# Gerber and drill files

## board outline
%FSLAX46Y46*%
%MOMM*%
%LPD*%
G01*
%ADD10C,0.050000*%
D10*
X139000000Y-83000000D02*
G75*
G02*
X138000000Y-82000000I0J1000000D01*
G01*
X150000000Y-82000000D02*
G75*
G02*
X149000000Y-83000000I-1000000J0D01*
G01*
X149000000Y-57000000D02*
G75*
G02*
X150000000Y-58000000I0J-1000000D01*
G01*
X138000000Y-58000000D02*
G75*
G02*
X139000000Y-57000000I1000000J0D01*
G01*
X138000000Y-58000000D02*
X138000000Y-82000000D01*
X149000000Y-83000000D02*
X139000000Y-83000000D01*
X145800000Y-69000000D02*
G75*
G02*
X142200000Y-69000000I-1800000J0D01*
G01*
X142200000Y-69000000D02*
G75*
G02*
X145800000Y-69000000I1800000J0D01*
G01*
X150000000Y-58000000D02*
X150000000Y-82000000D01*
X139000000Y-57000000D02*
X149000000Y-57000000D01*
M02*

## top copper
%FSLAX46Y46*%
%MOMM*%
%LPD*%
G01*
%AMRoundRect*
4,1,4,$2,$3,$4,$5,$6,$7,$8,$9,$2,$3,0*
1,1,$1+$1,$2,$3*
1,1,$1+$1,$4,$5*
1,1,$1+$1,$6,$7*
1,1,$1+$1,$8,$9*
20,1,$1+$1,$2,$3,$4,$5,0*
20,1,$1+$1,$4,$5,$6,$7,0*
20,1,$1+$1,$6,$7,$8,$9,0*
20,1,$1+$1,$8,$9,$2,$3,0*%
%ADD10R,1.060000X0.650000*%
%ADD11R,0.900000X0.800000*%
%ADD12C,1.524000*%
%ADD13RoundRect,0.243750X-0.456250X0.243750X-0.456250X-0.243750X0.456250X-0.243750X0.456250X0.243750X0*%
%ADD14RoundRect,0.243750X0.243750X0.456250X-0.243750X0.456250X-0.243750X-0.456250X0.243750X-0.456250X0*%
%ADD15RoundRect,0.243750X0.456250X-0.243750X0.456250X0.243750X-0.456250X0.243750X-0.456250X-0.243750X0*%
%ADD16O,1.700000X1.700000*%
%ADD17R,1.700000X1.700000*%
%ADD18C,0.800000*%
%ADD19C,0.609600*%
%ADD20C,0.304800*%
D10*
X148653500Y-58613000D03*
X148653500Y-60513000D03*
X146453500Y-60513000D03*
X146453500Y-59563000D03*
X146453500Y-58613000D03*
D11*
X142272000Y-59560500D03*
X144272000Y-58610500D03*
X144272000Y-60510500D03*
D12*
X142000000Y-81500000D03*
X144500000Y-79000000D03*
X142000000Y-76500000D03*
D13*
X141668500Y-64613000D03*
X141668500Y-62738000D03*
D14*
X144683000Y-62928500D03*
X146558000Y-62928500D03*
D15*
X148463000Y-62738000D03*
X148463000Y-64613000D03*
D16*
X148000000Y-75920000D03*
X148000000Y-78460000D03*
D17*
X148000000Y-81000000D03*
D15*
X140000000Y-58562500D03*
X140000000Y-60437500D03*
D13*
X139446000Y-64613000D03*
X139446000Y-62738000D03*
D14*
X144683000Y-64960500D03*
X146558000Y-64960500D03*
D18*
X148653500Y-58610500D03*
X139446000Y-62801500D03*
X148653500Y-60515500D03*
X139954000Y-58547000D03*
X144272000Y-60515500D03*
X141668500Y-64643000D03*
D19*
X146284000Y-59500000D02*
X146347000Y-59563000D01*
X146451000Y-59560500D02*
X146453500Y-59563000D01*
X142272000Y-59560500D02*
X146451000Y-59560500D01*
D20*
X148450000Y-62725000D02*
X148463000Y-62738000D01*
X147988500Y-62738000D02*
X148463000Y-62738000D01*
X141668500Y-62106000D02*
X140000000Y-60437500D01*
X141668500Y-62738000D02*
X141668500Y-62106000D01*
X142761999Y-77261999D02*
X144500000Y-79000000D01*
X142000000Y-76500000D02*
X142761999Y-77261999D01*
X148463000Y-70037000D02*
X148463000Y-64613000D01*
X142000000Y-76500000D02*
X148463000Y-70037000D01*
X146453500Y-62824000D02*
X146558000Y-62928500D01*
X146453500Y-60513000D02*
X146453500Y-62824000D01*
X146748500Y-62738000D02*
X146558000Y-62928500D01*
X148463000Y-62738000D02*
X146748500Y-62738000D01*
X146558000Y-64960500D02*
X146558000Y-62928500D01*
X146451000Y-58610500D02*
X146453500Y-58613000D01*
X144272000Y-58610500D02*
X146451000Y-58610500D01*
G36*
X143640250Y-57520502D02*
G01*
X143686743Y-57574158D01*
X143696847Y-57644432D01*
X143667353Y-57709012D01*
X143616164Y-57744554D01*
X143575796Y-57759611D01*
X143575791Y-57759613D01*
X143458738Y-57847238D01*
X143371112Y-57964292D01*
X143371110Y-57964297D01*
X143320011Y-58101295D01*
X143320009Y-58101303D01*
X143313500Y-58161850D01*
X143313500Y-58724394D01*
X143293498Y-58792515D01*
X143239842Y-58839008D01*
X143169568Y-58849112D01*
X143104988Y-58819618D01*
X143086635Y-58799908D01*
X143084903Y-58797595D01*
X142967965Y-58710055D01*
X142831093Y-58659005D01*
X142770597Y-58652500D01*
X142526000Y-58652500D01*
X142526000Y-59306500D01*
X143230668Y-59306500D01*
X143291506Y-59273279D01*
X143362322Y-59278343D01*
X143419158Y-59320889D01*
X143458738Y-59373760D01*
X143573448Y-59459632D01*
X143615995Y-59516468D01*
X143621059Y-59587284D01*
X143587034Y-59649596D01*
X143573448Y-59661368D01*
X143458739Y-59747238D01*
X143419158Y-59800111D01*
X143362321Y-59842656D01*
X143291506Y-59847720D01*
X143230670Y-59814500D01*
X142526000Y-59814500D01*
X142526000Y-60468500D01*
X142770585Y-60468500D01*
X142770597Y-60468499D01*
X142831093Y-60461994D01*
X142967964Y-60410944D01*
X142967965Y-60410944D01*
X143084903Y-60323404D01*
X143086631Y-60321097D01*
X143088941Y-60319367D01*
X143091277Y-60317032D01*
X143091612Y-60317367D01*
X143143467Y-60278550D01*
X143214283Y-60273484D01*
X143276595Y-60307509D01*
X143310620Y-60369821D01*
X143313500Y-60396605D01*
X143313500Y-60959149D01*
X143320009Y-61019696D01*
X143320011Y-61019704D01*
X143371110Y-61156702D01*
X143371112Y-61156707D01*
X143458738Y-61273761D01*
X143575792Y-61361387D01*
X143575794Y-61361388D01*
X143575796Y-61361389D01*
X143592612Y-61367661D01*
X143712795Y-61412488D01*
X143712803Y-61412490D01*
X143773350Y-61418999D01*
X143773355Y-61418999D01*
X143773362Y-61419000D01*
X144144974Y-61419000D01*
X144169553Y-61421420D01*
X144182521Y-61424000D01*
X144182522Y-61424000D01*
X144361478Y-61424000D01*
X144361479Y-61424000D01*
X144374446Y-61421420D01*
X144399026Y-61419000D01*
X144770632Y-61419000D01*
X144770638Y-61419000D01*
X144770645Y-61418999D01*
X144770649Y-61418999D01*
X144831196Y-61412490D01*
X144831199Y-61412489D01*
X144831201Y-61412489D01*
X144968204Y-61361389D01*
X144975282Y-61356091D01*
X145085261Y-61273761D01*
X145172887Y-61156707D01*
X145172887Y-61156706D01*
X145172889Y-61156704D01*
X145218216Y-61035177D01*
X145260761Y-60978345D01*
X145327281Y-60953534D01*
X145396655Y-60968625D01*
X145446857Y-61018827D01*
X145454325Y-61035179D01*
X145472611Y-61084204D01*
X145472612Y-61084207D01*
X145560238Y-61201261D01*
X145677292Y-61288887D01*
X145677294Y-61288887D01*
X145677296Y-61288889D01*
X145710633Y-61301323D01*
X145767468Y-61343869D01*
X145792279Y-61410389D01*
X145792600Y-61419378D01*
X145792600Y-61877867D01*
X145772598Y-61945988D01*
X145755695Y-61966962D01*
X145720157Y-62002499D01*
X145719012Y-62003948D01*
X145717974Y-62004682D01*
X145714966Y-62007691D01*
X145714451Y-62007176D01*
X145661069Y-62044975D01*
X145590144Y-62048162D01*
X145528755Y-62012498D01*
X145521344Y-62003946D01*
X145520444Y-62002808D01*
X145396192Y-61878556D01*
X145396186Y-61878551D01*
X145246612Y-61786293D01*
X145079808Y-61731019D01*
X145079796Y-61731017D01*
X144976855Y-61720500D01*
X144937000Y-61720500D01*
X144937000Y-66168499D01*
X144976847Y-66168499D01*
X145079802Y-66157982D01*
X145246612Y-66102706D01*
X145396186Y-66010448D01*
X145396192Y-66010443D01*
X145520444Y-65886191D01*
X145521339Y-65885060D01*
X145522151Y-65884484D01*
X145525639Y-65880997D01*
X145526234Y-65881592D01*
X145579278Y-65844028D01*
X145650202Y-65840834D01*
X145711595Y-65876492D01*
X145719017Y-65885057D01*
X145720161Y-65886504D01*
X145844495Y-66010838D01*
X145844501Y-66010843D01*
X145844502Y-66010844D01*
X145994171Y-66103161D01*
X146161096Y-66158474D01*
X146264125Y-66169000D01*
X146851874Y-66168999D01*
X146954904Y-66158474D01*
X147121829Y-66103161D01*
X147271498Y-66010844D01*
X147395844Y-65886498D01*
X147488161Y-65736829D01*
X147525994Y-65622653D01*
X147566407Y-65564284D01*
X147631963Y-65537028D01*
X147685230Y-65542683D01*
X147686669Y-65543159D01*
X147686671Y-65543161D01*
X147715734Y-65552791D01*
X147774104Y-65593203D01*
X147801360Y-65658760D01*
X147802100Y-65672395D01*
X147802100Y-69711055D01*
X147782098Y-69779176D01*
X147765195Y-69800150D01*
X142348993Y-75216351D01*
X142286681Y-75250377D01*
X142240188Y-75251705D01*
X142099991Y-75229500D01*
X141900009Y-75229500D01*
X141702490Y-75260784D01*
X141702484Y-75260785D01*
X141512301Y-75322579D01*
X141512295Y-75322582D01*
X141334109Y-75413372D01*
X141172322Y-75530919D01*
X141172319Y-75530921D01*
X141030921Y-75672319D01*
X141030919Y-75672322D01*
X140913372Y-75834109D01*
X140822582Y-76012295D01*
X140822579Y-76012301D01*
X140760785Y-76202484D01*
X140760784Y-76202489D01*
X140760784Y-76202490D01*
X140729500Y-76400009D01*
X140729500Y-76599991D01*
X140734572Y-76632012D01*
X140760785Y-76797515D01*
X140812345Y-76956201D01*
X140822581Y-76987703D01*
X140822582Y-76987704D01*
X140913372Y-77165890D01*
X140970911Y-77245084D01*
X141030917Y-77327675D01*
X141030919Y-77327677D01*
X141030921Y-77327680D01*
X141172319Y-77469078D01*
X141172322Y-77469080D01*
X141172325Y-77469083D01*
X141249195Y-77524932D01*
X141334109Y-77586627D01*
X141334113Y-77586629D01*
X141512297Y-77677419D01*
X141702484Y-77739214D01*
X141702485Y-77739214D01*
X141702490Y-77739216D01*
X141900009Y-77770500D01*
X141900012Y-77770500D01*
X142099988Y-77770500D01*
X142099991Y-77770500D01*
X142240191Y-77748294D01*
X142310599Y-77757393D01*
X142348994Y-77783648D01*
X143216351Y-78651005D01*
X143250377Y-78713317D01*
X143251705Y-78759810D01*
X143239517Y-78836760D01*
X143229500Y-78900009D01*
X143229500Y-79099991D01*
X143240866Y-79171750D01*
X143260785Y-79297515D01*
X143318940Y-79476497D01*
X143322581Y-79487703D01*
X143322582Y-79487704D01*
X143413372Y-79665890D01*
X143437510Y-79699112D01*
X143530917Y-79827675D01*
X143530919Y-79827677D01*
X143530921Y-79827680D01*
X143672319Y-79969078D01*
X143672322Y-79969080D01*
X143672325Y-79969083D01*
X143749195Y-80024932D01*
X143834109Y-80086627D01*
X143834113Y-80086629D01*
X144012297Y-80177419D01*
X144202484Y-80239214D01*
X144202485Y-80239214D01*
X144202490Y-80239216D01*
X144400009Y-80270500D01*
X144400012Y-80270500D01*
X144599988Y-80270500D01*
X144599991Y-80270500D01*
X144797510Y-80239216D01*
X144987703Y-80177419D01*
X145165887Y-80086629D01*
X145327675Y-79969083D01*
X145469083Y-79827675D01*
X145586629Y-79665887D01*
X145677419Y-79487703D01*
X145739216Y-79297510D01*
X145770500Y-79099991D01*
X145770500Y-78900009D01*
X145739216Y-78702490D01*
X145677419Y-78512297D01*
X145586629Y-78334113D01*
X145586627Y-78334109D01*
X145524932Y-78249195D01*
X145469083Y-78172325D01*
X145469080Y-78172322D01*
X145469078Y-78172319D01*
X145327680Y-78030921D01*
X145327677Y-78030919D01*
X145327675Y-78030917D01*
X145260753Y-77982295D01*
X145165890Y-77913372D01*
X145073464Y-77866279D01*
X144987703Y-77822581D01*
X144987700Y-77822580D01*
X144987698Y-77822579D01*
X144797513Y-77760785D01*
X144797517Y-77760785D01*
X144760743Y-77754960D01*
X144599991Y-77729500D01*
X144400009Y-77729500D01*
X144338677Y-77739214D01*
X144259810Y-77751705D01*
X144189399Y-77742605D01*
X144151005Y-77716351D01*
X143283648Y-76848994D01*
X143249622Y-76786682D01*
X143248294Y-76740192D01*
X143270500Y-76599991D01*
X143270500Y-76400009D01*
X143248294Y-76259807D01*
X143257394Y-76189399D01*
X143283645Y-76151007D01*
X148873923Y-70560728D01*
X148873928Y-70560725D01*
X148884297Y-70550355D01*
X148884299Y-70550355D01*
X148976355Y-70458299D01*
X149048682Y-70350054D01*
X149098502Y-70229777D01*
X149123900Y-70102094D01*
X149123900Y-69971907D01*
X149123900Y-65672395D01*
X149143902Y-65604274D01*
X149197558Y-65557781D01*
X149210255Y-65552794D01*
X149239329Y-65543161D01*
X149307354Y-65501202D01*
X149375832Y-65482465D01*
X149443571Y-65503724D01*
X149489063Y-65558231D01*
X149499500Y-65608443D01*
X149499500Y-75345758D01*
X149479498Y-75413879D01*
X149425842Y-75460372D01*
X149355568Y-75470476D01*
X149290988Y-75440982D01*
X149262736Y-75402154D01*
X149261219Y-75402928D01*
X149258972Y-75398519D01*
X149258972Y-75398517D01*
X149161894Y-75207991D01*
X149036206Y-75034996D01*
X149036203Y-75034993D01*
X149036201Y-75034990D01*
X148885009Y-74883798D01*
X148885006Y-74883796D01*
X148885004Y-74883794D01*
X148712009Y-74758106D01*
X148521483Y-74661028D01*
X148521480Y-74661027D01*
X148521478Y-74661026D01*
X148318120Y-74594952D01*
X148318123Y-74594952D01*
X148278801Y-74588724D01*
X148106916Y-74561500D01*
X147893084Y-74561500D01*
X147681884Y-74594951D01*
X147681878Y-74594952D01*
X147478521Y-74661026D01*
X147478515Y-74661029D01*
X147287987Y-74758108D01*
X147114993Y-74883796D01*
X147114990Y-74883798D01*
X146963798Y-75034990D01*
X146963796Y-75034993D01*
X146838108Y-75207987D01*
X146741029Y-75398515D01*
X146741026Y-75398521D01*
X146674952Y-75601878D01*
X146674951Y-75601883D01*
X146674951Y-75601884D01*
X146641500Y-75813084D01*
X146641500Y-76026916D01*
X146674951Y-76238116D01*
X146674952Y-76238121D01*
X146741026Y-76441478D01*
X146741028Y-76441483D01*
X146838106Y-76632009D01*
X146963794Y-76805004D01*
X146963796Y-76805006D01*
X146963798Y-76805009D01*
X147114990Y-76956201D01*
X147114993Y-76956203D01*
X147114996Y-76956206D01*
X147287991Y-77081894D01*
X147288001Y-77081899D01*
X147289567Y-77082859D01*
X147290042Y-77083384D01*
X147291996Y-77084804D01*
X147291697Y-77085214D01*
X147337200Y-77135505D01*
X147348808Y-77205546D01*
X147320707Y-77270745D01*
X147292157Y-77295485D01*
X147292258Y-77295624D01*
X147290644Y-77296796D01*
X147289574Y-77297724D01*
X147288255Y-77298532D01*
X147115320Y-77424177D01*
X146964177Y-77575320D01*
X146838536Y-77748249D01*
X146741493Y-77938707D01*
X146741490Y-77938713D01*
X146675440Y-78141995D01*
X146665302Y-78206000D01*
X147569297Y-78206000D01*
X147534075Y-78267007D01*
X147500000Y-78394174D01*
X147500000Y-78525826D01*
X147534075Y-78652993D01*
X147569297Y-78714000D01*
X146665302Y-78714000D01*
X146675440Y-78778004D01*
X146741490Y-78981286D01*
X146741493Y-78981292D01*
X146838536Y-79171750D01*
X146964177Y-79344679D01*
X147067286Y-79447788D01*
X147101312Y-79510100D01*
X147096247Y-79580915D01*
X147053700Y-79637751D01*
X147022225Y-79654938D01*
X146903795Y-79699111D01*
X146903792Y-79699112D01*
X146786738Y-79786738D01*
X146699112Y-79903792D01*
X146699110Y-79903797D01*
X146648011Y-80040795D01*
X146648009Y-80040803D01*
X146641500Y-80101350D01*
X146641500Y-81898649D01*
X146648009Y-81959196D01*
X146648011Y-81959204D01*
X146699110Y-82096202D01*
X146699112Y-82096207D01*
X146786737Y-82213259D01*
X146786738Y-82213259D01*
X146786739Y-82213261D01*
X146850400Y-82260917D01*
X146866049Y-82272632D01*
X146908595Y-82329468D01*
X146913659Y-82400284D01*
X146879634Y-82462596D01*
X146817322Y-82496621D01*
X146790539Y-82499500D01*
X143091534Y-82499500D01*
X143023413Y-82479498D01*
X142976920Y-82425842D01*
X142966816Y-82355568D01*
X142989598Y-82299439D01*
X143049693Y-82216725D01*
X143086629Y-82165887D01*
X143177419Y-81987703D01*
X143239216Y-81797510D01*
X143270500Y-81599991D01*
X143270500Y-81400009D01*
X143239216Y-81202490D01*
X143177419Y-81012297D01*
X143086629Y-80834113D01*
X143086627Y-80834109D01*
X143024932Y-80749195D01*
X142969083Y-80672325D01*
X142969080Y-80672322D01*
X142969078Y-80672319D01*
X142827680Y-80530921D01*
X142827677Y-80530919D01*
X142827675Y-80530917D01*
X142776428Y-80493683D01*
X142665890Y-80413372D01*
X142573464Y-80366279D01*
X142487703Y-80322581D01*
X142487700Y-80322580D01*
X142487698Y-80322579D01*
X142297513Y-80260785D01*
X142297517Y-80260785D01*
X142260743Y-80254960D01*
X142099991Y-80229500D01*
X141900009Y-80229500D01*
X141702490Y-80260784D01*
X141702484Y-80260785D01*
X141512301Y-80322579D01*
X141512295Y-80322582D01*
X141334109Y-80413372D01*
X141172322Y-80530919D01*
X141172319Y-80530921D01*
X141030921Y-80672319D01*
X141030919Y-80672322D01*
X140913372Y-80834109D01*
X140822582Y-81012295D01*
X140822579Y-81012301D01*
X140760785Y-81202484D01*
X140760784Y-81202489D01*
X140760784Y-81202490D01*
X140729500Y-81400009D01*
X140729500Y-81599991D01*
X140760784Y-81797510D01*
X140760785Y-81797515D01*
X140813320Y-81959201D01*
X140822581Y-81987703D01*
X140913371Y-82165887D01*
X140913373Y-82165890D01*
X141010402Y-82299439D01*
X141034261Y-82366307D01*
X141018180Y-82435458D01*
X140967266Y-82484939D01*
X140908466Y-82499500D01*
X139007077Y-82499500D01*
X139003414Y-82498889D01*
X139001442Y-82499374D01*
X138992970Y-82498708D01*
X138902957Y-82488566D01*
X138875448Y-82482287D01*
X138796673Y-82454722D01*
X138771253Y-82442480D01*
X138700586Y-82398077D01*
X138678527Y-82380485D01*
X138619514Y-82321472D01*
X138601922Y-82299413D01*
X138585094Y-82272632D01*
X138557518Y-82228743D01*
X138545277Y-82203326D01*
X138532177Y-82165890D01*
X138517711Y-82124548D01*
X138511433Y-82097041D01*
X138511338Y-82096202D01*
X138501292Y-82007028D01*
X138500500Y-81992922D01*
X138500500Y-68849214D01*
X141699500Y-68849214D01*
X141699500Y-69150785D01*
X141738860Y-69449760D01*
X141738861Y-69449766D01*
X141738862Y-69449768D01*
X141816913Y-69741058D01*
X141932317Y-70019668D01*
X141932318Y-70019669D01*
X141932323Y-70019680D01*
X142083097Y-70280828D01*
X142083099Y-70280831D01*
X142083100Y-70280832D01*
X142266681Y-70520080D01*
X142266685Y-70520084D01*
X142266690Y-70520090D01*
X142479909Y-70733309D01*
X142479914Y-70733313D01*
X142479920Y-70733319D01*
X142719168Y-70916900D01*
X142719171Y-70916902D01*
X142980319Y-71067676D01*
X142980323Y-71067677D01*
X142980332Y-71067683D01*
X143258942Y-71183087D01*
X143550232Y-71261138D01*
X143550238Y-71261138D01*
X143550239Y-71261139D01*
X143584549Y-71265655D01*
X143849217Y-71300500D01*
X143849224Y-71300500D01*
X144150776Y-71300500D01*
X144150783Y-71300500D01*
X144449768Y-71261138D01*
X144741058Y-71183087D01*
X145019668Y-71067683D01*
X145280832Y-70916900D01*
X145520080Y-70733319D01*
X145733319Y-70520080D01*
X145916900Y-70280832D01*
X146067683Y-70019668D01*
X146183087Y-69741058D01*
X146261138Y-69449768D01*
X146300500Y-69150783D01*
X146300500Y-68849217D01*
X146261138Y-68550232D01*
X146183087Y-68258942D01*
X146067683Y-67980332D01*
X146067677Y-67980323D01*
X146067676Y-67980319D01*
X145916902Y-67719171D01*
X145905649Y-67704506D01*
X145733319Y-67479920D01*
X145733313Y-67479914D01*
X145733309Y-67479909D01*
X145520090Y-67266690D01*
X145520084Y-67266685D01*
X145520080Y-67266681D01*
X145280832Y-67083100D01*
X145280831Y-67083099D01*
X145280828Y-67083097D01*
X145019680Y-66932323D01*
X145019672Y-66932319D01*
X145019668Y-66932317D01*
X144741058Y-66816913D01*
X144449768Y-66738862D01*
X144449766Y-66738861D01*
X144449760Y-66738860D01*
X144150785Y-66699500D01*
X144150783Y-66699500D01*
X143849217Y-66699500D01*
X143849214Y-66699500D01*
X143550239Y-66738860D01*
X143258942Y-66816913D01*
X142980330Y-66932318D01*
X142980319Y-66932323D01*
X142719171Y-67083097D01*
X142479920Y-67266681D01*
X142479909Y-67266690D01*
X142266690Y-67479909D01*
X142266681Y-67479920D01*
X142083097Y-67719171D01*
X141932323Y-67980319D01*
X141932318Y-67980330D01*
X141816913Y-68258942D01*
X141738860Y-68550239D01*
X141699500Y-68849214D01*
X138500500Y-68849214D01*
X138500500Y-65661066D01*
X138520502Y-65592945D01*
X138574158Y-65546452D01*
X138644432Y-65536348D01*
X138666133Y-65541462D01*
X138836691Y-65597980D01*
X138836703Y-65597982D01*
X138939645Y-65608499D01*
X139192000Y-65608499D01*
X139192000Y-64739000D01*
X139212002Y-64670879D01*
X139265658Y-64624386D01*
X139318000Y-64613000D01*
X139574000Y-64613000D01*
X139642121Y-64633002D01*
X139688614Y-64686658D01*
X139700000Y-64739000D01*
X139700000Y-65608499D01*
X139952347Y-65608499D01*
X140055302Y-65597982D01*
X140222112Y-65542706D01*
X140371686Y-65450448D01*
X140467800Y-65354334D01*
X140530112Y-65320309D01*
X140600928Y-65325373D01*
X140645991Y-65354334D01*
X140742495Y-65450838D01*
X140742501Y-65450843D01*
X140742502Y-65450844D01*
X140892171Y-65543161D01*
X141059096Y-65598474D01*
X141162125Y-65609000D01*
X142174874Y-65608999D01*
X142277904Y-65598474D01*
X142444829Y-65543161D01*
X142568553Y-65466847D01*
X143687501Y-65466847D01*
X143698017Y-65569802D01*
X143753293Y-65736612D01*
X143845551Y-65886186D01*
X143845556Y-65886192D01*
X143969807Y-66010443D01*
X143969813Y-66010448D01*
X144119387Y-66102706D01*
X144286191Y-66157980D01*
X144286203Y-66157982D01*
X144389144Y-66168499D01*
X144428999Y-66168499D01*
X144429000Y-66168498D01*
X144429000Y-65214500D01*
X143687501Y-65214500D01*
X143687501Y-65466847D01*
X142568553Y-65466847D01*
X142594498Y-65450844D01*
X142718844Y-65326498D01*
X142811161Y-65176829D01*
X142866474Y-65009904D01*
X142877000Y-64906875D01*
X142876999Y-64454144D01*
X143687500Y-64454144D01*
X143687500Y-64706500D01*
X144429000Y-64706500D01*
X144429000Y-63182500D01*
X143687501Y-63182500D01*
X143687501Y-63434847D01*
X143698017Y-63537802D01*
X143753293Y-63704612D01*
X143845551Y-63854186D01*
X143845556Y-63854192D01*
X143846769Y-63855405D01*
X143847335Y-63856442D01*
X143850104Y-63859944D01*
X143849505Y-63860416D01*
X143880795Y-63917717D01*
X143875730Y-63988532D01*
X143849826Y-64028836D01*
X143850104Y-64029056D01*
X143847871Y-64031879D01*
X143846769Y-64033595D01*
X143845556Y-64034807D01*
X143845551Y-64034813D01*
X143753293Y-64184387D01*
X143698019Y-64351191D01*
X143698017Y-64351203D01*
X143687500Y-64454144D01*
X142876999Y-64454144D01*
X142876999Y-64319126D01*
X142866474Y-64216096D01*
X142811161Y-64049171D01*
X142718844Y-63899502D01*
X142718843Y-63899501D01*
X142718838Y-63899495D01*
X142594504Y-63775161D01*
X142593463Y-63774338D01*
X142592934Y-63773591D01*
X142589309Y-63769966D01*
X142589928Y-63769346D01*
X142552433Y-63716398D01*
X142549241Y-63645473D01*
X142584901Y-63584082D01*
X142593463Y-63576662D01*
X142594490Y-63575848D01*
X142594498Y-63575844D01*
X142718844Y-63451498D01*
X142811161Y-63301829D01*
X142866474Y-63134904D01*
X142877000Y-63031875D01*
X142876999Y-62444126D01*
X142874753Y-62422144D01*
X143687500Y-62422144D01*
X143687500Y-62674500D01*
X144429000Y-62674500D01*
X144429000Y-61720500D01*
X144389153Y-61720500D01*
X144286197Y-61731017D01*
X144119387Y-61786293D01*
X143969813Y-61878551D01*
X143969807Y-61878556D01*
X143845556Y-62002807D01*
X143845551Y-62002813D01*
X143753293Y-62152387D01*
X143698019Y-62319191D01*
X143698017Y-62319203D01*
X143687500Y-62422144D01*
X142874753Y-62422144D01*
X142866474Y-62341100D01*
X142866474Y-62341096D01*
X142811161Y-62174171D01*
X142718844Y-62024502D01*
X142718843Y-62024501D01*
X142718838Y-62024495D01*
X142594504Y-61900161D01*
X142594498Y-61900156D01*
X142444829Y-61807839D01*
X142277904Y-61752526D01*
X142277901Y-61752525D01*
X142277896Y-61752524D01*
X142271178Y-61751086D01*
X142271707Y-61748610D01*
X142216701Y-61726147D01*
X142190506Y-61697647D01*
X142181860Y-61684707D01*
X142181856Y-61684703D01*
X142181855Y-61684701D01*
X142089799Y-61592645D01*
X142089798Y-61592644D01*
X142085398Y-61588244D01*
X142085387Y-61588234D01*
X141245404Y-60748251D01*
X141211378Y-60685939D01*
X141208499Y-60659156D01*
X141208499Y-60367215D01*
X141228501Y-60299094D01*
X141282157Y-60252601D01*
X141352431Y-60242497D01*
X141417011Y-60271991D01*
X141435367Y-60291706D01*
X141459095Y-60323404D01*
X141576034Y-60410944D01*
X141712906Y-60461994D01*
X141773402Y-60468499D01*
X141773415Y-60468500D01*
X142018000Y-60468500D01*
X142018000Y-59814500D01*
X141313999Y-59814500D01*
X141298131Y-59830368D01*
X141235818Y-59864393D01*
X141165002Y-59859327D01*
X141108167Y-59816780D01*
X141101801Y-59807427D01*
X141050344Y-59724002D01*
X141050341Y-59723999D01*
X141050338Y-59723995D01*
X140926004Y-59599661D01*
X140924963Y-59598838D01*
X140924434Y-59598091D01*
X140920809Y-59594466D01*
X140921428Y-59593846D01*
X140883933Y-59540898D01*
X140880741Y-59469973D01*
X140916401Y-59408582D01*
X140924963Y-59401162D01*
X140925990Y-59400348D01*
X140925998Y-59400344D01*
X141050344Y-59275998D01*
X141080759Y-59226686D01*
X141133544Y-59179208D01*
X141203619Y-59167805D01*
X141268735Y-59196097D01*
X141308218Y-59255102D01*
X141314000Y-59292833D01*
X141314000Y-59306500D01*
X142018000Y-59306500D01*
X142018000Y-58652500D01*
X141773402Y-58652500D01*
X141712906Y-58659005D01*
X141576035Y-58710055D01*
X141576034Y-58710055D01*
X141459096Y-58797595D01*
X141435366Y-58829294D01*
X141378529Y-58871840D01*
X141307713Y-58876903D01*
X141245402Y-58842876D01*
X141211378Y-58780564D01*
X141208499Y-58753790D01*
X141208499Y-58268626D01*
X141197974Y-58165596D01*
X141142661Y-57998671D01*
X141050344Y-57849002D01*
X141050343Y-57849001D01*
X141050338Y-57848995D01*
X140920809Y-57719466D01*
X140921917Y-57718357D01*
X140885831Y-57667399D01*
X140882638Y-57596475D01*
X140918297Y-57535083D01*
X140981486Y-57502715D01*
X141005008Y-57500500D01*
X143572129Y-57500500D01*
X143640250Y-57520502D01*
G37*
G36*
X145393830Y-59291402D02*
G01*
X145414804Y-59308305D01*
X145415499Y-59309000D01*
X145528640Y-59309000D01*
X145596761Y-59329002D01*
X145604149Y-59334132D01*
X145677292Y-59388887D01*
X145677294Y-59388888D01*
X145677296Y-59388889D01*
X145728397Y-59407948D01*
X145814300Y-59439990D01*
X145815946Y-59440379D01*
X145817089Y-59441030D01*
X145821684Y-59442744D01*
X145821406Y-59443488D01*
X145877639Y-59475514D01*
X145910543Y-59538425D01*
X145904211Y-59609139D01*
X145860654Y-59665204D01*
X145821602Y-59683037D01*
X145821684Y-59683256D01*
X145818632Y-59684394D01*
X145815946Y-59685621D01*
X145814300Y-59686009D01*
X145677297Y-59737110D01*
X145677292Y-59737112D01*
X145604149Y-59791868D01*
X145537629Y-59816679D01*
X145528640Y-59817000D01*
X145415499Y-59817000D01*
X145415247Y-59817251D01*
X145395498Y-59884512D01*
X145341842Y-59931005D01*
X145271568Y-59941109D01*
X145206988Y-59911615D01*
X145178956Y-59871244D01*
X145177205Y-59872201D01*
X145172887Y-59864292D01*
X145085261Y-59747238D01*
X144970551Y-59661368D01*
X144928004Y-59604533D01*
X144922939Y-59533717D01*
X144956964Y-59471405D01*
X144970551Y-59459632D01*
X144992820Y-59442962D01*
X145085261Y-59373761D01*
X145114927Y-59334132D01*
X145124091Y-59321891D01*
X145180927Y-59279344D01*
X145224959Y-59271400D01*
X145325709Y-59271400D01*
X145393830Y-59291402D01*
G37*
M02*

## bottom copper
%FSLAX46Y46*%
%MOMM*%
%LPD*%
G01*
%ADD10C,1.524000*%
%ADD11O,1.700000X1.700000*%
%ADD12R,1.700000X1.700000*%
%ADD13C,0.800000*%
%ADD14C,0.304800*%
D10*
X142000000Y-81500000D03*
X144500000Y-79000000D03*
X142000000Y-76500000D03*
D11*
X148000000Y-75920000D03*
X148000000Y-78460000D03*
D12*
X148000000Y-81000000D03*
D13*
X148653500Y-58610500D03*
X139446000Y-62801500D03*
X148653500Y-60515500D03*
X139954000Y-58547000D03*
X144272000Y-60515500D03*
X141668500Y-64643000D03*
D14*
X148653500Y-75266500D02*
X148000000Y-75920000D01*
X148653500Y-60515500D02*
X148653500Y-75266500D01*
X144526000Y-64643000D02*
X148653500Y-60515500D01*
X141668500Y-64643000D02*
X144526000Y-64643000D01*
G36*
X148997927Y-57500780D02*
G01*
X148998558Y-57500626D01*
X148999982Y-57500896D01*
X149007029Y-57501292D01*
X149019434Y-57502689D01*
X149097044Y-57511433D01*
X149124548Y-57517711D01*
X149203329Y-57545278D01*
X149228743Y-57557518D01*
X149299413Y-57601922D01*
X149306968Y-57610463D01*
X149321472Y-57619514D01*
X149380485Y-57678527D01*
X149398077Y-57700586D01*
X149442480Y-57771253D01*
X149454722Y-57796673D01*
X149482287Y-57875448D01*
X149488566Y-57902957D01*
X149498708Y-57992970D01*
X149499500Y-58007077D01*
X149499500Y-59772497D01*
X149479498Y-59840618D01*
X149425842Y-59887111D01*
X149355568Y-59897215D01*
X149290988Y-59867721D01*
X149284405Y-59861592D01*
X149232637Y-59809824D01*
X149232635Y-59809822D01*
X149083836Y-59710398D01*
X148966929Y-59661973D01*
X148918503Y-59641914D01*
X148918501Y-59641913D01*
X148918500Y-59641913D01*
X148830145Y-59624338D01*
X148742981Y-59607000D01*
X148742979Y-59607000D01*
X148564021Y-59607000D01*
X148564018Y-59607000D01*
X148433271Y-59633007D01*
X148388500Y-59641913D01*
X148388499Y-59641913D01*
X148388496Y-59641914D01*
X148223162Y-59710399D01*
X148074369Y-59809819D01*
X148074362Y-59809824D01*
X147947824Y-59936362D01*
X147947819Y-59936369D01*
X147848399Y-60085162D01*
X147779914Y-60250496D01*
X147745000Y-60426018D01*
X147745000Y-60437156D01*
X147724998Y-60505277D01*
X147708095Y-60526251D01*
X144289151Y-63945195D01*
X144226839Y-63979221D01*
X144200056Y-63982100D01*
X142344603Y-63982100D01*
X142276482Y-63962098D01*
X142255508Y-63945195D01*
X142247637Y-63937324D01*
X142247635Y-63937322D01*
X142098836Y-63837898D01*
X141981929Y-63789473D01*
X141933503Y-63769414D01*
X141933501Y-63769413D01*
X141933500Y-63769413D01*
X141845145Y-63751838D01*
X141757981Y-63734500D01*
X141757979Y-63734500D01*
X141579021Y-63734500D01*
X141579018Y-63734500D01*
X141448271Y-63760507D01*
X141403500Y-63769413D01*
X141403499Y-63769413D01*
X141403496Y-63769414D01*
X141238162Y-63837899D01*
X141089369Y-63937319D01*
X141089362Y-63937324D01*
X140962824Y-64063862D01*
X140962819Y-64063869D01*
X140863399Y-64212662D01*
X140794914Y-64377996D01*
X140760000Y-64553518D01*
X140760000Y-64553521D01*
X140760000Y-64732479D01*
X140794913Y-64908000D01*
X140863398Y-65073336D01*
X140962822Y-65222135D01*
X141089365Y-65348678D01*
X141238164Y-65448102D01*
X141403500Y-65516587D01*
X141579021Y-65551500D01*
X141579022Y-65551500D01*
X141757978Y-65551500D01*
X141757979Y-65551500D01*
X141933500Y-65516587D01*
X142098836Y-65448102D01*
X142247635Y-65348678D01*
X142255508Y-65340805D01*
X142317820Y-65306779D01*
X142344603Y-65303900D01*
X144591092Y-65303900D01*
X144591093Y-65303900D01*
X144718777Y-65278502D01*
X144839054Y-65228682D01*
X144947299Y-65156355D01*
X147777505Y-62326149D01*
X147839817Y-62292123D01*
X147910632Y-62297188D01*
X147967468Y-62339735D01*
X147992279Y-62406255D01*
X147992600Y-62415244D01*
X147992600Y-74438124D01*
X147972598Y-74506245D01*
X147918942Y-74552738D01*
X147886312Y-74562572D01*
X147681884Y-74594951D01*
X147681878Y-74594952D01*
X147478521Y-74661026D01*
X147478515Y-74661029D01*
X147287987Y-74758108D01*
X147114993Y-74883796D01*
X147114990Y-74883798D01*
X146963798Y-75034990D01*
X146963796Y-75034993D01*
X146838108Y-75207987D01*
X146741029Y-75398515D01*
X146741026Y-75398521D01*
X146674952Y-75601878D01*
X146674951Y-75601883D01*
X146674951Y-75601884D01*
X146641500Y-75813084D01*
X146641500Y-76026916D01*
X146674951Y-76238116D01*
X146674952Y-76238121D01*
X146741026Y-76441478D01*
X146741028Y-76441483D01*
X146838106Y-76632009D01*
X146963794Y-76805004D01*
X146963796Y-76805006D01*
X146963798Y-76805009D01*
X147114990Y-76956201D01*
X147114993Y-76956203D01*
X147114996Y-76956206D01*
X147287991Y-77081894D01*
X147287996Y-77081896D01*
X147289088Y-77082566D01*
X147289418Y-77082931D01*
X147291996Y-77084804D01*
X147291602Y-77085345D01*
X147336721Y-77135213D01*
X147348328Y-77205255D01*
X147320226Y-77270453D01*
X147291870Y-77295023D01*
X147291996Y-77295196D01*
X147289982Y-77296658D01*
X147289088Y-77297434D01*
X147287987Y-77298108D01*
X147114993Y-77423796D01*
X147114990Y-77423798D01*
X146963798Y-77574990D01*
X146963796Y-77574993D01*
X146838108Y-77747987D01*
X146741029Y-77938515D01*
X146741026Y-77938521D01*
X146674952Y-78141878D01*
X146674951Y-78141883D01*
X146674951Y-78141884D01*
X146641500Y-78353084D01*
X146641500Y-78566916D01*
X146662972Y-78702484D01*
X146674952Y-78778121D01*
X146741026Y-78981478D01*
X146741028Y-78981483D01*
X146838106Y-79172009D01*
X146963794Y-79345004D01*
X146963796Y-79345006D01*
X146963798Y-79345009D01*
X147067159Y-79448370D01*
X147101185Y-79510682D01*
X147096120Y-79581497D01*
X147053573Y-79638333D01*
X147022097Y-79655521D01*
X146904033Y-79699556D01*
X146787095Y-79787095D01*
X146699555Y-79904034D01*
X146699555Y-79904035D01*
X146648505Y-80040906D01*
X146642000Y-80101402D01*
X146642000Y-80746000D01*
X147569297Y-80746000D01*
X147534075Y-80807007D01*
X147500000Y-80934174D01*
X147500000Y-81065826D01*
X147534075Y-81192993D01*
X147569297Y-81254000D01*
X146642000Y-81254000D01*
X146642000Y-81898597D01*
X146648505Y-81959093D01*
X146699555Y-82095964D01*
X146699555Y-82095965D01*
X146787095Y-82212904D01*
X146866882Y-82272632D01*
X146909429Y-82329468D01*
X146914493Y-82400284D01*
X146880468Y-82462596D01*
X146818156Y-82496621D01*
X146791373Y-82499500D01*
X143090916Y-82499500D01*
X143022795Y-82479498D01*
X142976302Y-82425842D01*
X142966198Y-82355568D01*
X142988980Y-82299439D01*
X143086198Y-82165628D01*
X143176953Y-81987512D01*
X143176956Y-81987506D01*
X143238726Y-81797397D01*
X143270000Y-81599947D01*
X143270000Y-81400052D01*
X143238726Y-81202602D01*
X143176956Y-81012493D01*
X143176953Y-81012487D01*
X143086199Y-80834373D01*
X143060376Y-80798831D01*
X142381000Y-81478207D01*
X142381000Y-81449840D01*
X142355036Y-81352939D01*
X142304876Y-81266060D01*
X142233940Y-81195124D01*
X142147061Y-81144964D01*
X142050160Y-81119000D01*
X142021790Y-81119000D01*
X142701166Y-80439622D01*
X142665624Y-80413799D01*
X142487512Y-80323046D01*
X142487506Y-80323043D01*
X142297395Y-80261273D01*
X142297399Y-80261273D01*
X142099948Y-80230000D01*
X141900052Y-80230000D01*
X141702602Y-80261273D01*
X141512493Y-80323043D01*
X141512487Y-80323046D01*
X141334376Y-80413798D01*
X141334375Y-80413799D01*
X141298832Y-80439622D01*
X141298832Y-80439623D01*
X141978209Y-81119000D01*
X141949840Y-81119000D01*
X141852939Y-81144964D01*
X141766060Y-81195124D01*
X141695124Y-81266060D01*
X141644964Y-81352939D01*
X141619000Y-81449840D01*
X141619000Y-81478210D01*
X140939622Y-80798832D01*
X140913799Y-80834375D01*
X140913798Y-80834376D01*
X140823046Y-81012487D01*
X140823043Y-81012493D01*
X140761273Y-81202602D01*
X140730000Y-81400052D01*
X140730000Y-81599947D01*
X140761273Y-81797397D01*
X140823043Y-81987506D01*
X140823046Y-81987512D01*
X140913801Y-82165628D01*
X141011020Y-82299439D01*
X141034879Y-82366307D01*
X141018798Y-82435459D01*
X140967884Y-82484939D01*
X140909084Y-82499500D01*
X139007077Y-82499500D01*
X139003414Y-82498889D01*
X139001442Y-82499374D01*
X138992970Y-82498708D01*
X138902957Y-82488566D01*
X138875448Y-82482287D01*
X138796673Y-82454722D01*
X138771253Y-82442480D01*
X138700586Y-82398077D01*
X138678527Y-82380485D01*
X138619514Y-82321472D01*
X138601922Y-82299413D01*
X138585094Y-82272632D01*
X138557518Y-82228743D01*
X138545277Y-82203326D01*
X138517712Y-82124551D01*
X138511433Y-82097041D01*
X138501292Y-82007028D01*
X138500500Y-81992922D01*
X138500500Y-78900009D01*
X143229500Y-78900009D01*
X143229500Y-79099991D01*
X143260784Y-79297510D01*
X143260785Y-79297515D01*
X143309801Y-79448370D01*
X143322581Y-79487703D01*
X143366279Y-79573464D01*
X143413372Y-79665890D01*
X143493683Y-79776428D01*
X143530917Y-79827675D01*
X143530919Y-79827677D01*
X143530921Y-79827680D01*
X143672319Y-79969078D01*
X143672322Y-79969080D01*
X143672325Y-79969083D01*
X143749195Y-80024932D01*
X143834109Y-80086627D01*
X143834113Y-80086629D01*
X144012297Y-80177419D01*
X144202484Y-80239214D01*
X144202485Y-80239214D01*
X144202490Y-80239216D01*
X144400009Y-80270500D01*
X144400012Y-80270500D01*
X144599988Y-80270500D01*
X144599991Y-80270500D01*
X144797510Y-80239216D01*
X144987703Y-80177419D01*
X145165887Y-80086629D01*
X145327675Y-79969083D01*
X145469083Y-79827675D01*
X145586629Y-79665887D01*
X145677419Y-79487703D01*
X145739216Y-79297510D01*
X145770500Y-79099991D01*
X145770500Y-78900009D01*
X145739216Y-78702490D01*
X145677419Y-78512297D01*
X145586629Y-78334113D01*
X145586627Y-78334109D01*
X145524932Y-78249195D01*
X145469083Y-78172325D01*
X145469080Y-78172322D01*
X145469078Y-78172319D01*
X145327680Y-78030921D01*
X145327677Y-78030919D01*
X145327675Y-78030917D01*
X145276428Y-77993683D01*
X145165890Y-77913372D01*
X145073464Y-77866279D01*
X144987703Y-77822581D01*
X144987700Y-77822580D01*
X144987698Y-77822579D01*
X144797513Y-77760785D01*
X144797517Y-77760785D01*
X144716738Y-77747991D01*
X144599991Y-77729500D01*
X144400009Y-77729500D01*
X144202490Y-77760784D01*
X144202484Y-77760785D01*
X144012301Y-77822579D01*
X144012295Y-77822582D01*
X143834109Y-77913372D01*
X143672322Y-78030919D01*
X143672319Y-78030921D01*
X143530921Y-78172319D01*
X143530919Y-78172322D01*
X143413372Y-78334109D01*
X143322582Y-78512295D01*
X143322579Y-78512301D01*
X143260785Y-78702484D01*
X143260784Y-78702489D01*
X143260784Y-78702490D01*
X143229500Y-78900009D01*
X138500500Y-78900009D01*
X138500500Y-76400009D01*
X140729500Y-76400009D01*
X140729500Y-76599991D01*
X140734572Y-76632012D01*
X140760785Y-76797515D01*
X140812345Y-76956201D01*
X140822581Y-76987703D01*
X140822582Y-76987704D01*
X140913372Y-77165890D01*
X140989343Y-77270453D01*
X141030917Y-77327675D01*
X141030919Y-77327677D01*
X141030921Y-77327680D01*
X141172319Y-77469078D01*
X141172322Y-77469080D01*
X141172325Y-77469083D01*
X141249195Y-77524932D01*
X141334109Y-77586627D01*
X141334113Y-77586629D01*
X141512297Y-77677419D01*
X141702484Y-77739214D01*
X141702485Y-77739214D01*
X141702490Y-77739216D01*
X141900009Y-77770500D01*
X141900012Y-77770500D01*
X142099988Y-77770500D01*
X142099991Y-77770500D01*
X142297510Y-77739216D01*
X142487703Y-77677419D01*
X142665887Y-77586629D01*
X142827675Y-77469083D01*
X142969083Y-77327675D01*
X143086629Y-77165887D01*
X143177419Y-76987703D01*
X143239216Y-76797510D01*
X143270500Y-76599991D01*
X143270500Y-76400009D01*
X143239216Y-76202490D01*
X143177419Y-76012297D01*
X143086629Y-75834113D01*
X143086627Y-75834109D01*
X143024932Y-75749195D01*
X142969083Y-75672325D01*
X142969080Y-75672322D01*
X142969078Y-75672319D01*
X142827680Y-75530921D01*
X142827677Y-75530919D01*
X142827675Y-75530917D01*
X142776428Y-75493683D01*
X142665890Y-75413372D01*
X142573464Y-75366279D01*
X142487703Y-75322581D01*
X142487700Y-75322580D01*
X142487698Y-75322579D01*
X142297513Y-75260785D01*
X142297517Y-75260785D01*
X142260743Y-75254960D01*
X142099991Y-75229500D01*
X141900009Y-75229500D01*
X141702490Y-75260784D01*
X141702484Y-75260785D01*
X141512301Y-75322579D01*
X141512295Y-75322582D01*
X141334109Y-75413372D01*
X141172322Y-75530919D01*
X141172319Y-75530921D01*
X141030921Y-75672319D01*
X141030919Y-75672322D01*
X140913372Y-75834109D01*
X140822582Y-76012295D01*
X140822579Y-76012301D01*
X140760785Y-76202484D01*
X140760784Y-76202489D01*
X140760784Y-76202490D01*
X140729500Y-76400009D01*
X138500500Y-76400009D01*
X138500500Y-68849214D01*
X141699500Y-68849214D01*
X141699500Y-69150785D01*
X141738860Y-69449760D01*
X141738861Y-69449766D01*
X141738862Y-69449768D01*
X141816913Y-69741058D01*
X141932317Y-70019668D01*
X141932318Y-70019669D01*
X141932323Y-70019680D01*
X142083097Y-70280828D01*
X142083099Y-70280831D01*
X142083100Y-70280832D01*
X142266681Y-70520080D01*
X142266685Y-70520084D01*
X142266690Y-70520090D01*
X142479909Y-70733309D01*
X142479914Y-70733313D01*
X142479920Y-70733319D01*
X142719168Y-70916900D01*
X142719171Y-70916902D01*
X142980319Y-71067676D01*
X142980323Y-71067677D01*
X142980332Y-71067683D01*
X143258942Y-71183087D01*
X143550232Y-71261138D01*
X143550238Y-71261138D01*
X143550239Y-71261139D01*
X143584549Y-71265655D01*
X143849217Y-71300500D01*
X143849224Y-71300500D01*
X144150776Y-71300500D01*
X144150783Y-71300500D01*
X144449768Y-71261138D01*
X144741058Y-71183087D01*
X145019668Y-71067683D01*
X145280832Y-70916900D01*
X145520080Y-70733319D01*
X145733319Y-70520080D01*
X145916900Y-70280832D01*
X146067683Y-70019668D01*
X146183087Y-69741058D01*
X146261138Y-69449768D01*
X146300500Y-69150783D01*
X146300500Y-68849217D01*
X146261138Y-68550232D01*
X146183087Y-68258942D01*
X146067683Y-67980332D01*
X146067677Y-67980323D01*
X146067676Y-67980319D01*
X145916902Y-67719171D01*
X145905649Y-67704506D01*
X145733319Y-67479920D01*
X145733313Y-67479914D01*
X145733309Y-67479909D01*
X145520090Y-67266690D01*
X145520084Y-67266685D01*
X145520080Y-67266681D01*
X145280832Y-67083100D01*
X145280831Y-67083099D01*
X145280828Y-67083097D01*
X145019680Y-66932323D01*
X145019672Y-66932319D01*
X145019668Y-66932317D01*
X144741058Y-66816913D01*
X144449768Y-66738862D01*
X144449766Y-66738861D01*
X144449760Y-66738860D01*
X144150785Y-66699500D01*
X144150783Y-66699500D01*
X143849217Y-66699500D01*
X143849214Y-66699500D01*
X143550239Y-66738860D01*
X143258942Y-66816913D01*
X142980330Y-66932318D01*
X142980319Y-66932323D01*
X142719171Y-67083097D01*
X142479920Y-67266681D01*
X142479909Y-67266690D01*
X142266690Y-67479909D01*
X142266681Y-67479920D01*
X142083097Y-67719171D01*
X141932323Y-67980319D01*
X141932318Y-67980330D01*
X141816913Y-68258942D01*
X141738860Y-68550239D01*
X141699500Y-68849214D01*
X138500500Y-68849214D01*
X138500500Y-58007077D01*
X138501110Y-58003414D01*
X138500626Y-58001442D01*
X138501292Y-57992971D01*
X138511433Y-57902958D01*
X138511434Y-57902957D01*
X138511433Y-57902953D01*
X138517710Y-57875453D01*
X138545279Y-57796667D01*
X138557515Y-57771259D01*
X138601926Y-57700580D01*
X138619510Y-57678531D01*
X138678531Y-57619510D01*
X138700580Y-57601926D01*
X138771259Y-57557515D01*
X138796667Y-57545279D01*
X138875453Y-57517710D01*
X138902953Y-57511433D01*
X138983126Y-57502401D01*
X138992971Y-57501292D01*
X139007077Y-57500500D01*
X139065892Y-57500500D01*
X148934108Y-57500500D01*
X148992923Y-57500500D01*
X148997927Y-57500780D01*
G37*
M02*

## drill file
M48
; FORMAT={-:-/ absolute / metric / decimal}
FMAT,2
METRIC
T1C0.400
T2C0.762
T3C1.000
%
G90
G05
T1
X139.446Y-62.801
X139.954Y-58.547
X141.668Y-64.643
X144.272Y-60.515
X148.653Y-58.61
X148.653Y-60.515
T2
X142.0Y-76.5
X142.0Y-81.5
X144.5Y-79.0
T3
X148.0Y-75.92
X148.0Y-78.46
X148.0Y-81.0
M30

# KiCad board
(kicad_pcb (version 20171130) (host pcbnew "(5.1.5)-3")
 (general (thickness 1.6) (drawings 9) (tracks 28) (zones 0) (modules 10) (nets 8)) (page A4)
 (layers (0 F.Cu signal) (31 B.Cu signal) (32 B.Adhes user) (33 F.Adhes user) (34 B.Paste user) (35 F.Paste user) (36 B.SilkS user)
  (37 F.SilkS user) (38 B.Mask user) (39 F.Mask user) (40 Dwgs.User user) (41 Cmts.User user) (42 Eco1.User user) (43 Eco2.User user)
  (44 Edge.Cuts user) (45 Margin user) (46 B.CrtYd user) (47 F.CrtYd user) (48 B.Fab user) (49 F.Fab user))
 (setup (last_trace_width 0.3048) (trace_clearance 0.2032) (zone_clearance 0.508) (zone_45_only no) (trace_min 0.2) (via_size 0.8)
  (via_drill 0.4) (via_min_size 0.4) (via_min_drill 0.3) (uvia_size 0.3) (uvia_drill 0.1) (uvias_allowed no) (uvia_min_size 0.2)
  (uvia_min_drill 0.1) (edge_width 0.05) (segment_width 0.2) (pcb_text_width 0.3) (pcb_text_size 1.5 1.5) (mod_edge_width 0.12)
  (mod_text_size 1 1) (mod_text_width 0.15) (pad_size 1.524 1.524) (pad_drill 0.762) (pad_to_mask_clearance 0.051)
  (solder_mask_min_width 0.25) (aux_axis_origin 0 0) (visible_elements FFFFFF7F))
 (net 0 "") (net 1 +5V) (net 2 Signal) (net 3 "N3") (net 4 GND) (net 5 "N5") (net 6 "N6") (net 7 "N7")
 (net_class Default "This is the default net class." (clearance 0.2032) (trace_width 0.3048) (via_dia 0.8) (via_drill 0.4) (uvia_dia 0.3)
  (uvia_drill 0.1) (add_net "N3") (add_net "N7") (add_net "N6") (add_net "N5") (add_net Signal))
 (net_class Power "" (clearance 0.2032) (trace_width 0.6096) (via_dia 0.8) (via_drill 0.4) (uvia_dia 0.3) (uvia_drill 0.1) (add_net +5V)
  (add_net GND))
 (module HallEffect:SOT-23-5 (layer F.Cu) (at 147.5535 59.563)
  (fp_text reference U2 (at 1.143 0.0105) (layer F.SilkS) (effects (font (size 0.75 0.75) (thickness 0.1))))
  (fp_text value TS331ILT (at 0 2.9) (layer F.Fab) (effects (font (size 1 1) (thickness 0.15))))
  (pad 5 smd rect (at 1.1 -0.95) (size 1.06 0.65) (layers F.Cu F.Paste F.Mask) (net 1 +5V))
  (pad 4 smd rect (at 1.1 0.95) (size 1.06 0.65) (layers F.Cu F.Paste F.Mask) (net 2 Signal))
  (pad 3 smd rect (at -1.1 0.95) (size 1.06 0.65) (layers F.Cu F.Paste F.Mask) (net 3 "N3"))
  (pad 2 smd rect (at -1.1 0) (size 1.06 0.65) (layers F.Cu F.Paste F.Mask) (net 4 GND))
  (pad 1 smd rect (at -1.1 -0.95) (size 1.06 0.65) (layers F.Cu F.Paste F.Mask) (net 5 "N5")))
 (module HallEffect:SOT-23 (layer F.Cu) (at 143.272 59.5605 180)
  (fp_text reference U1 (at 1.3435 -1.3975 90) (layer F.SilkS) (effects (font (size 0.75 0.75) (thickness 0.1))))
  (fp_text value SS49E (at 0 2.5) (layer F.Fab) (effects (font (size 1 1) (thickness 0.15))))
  (pad 3 smd rect (at 1 0 180) (size 0.9 0.8) (layers F.Cu F.Paste F.Mask) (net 4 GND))
  (pad 2 smd rect (at -1 0.95 180) (size 0.9 0.8) (layers F.Cu F.Paste F.Mask) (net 5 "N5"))
  (pad 1 smd rect (at -1 -0.95 180) (size 0.9 0.8) (layers F.Cu F.Paste F.Mask) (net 1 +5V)))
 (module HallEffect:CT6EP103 (layer F.Cu) (at 142 79 270)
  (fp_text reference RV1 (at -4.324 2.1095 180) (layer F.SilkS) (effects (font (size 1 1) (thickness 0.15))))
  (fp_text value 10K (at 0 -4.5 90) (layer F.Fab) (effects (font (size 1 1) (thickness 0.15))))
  (pad 3 thru_hole circle (at 2.5 0 270) (size 1.524 1.524) (drill 0.762) (layers *.Cu *.Mask) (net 1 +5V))
  (pad 2 thru_hole circle (at 0 -2.5 270) (size 1.524 1.524) (drill 0.762) (layers *.Cu *.Mask) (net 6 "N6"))
  (pad 1 thru_hole circle (at -2.5 0 270) (size 1.524 1.524) (drill 0.762) (layers *.Cu *.Mask) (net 6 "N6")))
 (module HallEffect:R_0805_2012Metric (layer F.Cu) (at 141.6685 63.6755 270)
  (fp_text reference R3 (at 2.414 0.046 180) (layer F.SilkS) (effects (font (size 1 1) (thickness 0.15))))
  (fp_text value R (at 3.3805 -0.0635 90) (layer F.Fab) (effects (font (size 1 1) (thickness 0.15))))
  (pad 2 smd roundrect (at 0.9375 0 270) (size 0.975 1.4) (layers F.Cu F.Paste F.Mask) (roundrect_rratio 0.25) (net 2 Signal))
  (pad 1 smd roundrect (at -0.9375 0 270) (size 0.975 1.4) (layers F.Cu F.Paste F.Mask) (roundrect_rratio 0.25) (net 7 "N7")))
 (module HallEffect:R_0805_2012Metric (layer F.Cu) (at 145.6205 62.9285 180)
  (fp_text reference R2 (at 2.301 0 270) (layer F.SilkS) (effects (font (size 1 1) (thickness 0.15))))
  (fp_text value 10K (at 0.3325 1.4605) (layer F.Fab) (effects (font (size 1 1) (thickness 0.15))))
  (pad 2 smd roundrect (at 0.9375 0 180) (size 0.975 1.4) (layers F.Cu F.Paste F.Mask) (roundrect_rratio 0.25) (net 4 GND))
  (pad 1 smd roundrect (at -0.9375 0 180) (size 0.975 1.4) (layers F.Cu F.Paste F.Mask) (roundrect_rratio 0.25) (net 3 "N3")))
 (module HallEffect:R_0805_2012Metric (layer F.Cu) (at 148.463 63.6755 90)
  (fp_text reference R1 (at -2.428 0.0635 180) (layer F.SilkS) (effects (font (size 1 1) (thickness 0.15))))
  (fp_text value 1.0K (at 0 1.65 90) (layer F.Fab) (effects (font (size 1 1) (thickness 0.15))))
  (pad 2 smd roundrect (at 0.9375 0 90) (size 0.975 1.4) (layers F.Cu F.Paste F.Mask) (roundrect_rratio 0.25) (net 3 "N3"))
  (pad 1 smd roundrect (at -0.9375 0 90) (size 0.975 1.4) (layers F.Cu F.Paste F.Mask) (roundrect_rratio 0.25) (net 6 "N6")))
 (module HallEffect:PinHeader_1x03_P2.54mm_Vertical (layer F.Cu) (at 148 81 180)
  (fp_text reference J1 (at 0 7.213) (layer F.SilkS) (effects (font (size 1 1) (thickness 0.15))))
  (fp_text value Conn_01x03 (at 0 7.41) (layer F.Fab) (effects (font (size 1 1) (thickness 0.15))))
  (pad 3 thru_hole oval (at 0 5.08 180) (size 1.7 1.7) (drill 1) (layers *.Cu *.Mask) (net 2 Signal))
  (pad 2 thru_hole oval (at 0 2.54 180) (size 1.7 1.7) (drill 1) (layers *.Cu *.Mask) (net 4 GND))
  (pad 1 thru_hole rect (at 0 0 180) (size 1.7 1.7) (drill 1) (layers *.Cu *.Mask) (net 1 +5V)))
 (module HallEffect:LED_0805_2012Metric (layer F.Cu) (at 140 59.5 90)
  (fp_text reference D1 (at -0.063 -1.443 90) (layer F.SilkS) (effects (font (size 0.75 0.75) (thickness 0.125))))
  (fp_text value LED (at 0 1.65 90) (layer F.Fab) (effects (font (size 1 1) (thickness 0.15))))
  (pad 2 smd roundrect (at 0.9375 0 90) (size 0.975 1.4) (layers F.Cu F.Paste F.Mask) (roundrect_rratio 0.25) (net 1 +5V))
  (pad 1 smd roundrect (at -0.9375 0 90) (size 0.975 1.4) (layers F.Cu F.Paste F.Mask) (roundrect_rratio 0.25) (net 7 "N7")))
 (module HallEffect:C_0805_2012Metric (layer F.Cu) (at 139.446 63.6755 270)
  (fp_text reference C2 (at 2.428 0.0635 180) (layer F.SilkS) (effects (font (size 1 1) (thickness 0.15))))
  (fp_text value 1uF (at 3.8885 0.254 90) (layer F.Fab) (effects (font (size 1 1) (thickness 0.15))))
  (pad 2 smd roundrect (at 0.9375 0 270) (size 0.975 1.4) (layers F.Cu F.Paste F.Mask) (roundrect_rratio 0.25) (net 4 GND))
  (pad 1 smd roundrect (at -0.9375 0 270) (size 0.975 1.4) (layers F.Cu F.Paste F.Mask) (roundrect_rratio 0.25) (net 1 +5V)))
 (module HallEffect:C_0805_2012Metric (layer F.Cu) (at 145.6205 64.9605 180)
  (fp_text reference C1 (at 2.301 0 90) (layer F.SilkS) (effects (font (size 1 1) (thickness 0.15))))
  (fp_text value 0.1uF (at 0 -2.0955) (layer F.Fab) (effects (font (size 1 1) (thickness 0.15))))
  (pad 2 smd roundrect (at 0.9375 0 180) (size 0.975 1.4) (layers F.Cu F.Paste F.Mask) (roundrect_rratio 0.25) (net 4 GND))
  (pad 1 smd roundrect (at -0.9375 0 180) (size 0.975 1.4) (layers F.Cu F.Paste F.Mask) (roundrect_rratio 0.25) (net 3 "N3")))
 (gr_arc (start 139 82) (end 138 82) (angle -90) (layer Edge.Cuts) (width 0.05))
 (gr_arc (start 149 82) (end 149 83) (angle -90) (layer Edge.Cuts) (width 0.05))
 (gr_arc (start 149 58) (end 150 58) (angle -90) (layer Edge.Cuts) (width 0.05))
 (gr_arc (start 139 58) (end 139 57) (angle -90) (layer Edge.Cuts) (width 0.05))
 (gr_line (start 138 58) (end 138 82) (layer Edge.Cuts) (width 0.05))
 (gr_line (start 149 83) (end 139 83) (layer Edge.Cuts) (width 0.05))
 (gr_circle (center 144 69) (end 145.8 69) (layer Edge.Cuts) (width 0.05))
 (gr_line (start 150 58) (end 150 82) (layer Edge.Cuts) (width 0.05))
 (gr_line (start 139 57) (end 149 57) (layer Edge.Cuts) (width 0.05))
 (via (at 148.6535 58.6105) (size 0.8) (drill 0.4) (layers F.Cu B.Cu) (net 1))
 (via (at 139.446 62.8015) (size 0.8) (drill 0.4) (layers F.Cu B.Cu) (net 1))
 (segment (start 146.284 59.5) (end 146.347 59.563) (width 0.6096) (layer F.Cu) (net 4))
 (segment (start 146.451 59.5605) (end 146.4535 59.563) (width 0.6096) (layer F.Cu) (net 4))
 (segment (start 142.272 59.5605) (end 146.451 59.5605) (width 0.6096) (layer F.Cu) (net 4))
 (via (at 148.6535 60.5155) (size 0.8) (drill 0.4) (layers F.Cu B.Cu) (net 2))
 (via (at 139.954 58.547) (size 0.8) (drill 0.4) (layers F.Cu B.Cu) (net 1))
 (via (at 144.272 60.5155) (size 0.8) (drill 0.4) (layers F.Cu B.Cu) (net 1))
 (segment (start 148.45 62.725) (end 148.463 62.738) (width 0.3048) (layer F.Cu) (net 3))
 (segment (start 147.9885 62.738) (end 148.463 62.738) (width 0.3048) (layer F.Cu) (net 3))
 (segment (start 141.6685 62.106) (end 140 60.4375) (width 0.3048) (layer F.Cu) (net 7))
 (segment (start 141.6685 62.738) (end 141.6685 62.106) (width 0.3048) (layer F.Cu) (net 7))
 (via (at 141.6685 64.643) (size 0.8) (drill 0.4) (layers F.Cu B.Cu) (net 2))
 (segment (start 142.761999 77.261999) (end 144.5 79) (width 0.3048) (layer F.Cu) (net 6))
 (segment (start 142 76.5) (end 142.761999 77.261999) (width 0.3048) (layer F.Cu) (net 6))
 (segment (start 148.463 70.037) (end 148.463 64.613) (width 0.3048) (layer F.Cu) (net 6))
 (segment (start 142 76.5) (end 148.463 70.037) (width 0.3048) (layer F.Cu) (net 6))
 (segment (start 146.4535 62.824) (end 146.558 62.9285) (width 0.3048) (layer F.Cu) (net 3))
 (segment (start 146.4535 60.513) (end 146.4535 62.824) (width 0.3048) (layer F.Cu) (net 3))
 (segment (start 146.7485 62.738) (end 146.558 62.9285) (width 0.3048) (layer F.Cu) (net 3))
 (segment (start 148.463 62.738) (end 146.7485 62.738) (width 0.3048) (layer F.Cu) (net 3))
 (segment (start 146.558 64.9605) (end 146.558 62.9285) (width 0.3048) (layer F.Cu) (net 3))
 (segment (start 148.6535 75.2665) (end 148 75.92) (width 0.3048) (layer B.Cu) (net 2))
 (segment (start 148.6535 60.5155) (end 148.6535 75.2665) (width 0.3048) (layer B.Cu) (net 2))
 (segment (start 144.526 64.643) (end 148.6535 60.5155) (width 0.3048) (layer B.Cu) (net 2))
 (segment (start 141.6685 64.643) (end 144.526 64.643) (width 0.3048) (layer B.Cu) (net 2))
 (segment (start 146.451 58.6105) (end 146.4535 58.613) (width 0.3048) (layer F.Cu) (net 5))
 (segment (start 144.272 58.6105) (end 146.451 58.6105) (width 0.3048) (layer F.Cu) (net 5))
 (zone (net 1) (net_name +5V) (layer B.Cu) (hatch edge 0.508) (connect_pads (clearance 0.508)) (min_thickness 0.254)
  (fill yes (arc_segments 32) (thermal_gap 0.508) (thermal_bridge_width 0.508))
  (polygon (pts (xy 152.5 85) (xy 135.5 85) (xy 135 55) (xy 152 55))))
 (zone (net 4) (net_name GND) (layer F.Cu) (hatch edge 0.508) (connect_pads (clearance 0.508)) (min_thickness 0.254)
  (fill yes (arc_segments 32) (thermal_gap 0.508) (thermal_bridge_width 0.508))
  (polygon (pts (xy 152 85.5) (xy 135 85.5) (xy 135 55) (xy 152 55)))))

